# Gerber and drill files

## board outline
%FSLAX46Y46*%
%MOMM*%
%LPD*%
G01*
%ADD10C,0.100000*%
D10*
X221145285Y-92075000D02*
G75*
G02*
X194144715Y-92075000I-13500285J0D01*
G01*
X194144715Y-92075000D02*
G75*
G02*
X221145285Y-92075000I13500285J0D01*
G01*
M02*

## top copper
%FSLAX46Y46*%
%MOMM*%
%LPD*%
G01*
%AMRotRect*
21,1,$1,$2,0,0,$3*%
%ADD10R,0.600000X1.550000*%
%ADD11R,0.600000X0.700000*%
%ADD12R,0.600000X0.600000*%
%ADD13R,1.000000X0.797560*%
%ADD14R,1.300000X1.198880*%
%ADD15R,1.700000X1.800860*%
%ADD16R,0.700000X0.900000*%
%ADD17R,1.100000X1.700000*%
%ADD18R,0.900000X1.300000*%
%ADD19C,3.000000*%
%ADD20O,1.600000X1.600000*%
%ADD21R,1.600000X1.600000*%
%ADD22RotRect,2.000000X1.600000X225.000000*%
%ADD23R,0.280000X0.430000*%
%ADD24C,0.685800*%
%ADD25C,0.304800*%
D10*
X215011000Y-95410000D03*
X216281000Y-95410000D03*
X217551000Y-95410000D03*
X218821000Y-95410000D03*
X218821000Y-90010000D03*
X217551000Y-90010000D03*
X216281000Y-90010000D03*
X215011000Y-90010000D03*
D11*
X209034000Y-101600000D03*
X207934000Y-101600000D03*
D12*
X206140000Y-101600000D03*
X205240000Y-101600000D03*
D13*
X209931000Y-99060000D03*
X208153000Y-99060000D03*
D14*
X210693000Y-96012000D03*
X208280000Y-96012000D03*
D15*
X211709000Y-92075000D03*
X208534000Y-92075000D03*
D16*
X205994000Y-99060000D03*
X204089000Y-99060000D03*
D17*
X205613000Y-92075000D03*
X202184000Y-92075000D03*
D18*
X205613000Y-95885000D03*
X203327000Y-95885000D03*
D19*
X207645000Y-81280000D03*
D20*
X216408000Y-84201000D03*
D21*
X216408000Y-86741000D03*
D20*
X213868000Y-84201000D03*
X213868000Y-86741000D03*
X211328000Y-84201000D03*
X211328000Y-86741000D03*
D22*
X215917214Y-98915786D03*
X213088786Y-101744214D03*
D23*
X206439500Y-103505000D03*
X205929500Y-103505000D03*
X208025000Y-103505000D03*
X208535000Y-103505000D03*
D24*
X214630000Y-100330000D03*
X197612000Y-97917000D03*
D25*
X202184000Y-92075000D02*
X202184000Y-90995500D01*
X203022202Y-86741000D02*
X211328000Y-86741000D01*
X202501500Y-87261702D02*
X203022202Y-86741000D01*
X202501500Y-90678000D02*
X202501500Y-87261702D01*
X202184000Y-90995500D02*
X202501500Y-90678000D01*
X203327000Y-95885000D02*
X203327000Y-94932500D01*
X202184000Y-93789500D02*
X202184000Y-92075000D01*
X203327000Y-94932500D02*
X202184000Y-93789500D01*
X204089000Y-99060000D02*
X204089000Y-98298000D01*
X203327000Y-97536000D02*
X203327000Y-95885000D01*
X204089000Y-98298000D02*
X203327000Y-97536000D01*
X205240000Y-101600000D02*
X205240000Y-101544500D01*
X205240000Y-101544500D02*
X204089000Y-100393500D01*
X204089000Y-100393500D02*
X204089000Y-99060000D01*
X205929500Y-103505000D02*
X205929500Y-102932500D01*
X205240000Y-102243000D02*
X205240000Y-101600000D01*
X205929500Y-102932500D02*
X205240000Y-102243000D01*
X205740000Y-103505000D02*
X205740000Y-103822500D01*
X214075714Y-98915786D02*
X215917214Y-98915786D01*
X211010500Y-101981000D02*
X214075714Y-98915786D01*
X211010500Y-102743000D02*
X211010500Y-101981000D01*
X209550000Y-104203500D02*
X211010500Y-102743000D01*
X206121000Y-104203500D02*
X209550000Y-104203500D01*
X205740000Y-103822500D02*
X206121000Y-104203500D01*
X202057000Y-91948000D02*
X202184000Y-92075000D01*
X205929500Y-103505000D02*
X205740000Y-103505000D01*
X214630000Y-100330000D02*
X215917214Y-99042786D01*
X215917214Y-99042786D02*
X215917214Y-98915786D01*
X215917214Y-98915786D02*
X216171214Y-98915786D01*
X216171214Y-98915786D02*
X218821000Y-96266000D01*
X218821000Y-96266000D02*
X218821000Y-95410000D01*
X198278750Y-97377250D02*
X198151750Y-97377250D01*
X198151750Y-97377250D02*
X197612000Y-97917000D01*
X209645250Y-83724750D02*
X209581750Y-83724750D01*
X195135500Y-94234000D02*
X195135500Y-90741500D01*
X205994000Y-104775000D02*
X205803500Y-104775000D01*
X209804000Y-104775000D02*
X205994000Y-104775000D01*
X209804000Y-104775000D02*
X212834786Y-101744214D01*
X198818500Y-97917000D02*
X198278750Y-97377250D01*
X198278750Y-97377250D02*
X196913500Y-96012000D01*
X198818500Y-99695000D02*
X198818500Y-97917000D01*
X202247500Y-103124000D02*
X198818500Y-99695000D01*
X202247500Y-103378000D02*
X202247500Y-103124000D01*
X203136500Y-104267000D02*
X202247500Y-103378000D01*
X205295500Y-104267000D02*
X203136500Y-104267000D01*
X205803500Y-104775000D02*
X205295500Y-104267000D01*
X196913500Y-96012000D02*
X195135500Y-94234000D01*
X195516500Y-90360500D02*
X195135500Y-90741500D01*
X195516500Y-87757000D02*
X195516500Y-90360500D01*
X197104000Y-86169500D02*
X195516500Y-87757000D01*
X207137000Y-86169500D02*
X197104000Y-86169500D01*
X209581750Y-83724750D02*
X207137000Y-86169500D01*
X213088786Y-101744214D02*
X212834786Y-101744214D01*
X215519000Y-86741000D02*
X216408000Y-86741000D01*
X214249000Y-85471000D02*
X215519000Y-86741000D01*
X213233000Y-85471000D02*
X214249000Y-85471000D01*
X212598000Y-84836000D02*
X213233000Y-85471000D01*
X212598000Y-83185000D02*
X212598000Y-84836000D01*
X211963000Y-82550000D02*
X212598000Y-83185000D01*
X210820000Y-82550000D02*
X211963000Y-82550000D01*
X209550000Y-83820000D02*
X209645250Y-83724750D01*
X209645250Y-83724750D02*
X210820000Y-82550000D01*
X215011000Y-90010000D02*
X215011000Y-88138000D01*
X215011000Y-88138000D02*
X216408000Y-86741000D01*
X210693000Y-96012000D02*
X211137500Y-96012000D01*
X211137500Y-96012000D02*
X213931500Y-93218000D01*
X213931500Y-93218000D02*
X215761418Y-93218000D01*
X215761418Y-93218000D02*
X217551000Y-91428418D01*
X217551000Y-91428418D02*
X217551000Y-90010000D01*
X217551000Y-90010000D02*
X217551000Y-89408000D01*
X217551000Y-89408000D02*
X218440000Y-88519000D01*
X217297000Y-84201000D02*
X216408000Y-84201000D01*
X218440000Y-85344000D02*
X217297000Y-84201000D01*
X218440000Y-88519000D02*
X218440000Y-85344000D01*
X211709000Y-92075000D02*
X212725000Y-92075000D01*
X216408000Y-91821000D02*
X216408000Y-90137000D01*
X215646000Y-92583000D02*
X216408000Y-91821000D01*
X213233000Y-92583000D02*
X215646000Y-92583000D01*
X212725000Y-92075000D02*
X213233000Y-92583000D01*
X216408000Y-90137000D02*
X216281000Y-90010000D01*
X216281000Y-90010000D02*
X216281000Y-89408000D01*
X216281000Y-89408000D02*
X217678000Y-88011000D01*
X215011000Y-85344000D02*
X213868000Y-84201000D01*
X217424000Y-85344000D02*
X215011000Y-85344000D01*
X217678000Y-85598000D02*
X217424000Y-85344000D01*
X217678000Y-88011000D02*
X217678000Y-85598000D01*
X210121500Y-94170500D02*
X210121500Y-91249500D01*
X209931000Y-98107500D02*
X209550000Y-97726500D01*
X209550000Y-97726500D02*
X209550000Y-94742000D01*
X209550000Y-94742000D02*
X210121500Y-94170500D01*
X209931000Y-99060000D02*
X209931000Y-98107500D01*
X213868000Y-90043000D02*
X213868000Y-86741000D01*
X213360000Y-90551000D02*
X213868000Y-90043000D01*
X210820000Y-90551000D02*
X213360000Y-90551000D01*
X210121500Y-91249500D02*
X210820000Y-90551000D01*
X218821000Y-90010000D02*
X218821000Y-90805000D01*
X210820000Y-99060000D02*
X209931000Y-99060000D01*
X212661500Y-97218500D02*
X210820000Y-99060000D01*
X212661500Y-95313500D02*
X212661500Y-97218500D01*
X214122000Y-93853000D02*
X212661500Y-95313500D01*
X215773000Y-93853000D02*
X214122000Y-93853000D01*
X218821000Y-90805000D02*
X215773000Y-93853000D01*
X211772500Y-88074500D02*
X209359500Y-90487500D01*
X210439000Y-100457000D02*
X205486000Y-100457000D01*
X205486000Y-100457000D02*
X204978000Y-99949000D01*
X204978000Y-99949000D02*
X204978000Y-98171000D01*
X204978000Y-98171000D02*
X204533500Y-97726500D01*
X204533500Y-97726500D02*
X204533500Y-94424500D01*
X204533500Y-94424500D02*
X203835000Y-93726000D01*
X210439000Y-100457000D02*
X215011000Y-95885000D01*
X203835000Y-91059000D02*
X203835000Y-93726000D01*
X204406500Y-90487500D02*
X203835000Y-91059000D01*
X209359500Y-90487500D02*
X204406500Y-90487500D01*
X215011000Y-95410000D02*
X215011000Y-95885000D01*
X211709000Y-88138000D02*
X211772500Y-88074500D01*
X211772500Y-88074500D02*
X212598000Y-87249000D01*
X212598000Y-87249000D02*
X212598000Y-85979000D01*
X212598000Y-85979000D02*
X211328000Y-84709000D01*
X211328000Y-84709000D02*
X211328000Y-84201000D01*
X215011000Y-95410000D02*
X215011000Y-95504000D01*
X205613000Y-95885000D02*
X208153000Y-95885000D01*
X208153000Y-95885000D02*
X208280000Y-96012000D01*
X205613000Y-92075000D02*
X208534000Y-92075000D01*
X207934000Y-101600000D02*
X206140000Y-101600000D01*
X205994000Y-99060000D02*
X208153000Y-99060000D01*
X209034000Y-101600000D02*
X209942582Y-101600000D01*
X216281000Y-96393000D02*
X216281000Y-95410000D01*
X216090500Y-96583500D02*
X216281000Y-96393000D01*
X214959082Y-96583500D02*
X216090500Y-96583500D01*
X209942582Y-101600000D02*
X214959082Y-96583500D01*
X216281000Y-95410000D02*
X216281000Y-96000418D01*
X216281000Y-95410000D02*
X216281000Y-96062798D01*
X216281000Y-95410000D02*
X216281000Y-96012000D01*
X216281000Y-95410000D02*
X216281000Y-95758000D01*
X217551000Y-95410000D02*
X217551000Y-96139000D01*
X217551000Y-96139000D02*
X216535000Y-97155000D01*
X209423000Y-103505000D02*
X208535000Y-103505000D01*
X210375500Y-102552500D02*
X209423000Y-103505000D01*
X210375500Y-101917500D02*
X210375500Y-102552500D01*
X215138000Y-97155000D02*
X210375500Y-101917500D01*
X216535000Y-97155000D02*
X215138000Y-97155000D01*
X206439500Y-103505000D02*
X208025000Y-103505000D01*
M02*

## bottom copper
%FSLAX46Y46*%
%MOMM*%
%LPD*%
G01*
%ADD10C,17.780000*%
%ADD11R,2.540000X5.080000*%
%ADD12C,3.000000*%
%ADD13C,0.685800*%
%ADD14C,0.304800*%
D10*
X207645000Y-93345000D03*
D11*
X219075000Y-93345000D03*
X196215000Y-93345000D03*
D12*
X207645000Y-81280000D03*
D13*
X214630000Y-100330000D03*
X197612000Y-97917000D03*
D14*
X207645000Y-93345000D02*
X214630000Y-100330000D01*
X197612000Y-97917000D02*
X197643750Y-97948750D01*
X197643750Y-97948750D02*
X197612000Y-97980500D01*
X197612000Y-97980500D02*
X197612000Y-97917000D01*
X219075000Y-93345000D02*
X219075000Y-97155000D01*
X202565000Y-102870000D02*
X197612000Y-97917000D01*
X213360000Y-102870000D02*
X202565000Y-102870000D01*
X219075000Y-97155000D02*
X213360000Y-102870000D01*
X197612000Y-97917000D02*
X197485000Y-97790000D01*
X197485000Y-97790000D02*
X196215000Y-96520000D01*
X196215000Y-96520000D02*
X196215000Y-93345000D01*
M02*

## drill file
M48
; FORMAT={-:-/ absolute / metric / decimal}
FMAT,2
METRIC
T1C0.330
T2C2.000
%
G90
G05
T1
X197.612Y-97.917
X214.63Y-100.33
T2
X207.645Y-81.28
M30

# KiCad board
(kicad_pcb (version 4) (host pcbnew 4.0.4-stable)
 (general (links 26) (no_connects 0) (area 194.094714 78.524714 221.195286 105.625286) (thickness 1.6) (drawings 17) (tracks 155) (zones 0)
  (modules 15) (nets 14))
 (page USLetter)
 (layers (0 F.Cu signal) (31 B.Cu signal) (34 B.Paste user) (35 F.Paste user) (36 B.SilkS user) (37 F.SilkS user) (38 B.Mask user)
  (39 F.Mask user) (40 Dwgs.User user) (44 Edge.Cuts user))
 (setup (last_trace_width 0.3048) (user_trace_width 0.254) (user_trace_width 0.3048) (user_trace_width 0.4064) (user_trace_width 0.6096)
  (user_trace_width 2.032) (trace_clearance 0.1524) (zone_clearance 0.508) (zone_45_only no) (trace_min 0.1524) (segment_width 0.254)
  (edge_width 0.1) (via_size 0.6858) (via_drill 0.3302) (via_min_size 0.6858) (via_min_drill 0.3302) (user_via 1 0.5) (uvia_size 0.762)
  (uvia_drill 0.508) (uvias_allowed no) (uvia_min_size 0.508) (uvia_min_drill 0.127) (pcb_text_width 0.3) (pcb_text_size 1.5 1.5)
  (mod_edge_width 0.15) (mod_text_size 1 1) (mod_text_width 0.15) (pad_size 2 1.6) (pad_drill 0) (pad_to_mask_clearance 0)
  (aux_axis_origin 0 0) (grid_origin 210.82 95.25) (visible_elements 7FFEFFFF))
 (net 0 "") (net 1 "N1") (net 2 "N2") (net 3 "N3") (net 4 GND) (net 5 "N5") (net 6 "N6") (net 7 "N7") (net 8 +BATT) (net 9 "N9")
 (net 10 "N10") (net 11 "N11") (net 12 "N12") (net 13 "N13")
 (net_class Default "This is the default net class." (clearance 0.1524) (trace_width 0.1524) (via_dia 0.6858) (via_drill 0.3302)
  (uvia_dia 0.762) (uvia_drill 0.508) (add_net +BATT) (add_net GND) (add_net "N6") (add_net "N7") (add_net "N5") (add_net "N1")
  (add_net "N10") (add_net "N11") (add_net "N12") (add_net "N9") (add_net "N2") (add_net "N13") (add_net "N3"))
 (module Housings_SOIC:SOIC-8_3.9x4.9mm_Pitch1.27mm (layer F.Cu) (at 216.916 92.71 90)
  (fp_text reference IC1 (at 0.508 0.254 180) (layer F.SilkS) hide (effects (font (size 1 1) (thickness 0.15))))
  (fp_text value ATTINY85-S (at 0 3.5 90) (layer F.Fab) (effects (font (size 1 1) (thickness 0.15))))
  (pad 1 smd rect (at -2.7 -1.905 90) (size 1.55 0.6) (layers F.Cu F.Paste F.Mask) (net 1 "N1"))
  (pad 2 smd rect (at -2.7 -0.635 90) (size 1.55 0.6) (layers F.Cu F.Paste F.Mask) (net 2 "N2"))
  (pad 3 smd rect (at -2.7 0.635 90) (size 1.55 0.6) (layers F.Cu F.Paste F.Mask) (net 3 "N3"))
  (pad 4 smd rect (at -2.7 1.905 90) (size 1.55 0.6) (layers F.Cu F.Paste F.Mask) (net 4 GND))
  (pad 5 smd rect (at 2.7 1.905 90) (size 1.55 0.6) (layers F.Cu F.Paste F.Mask) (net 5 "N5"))
  (pad 6 smd rect (at 2.7 0.635 90) (size 1.55 0.6) (layers F.Cu F.Paste F.Mask) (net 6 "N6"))
  (pad 7 smd rect (at 2.7 -0.635 90) (size 1.55 0.6) (layers F.Cu F.Paste F.Mask) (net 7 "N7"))
  (pad 8 smd rect (at 2.7 -1.905 90) (size 1.55 0.6) (layers F.Cu F.Paste F.Mask) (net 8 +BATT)))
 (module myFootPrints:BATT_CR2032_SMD (layer B.Cu) (at 207.645 93.345 180)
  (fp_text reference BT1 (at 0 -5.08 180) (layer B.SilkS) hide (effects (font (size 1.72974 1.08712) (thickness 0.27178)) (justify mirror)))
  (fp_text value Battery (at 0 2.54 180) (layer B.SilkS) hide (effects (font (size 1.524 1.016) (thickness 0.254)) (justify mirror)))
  (pad 2 smd circle (at 0 0 180) (size 17.78 17.78) (layers B.Cu B.Paste B.Mask) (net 4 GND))
  (pad 1 smd rect (at -11.43 0 180) (size 2.54 5.08) (layers B.Cu B.Paste B.Mask) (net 8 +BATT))
  (pad 1 smd rect (at 11.43 0 180) (size 2.54 5.08) (layers B.Cu B.Paste B.Mask) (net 8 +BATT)))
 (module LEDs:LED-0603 (layer F.Cu) (at 208.534 101.6)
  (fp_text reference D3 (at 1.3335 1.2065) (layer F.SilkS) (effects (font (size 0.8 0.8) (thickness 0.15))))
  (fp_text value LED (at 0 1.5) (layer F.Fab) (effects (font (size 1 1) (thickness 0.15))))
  (pad 2 smd rect (at 0.5 0 180) (size 0.6 0.7) (layers F.Cu F.Paste F.Mask) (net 2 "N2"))
  (pad 1 smd rect (at -0.6 0 180) (size 0.6 0.7) (layers F.Cu F.Paste F.Mask) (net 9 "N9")))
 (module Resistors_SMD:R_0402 (layer F.Cu) (at 205.74 101.6 180)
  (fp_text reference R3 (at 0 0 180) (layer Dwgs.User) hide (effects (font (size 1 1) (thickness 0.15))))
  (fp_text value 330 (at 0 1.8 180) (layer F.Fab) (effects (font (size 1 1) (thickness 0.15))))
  (pad 1 smd rect (at -0.4 0 180) (size 0.6 0.6) (layers F.Cu F.Paste F.Mask) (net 9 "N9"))
  (pad 2 smd rect (at 0.5 0 180) (size 0.6 0.6) (layers F.Cu F.Paste F.Mask) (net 4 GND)))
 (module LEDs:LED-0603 (layer F.Cu) (at 209.042 99.06)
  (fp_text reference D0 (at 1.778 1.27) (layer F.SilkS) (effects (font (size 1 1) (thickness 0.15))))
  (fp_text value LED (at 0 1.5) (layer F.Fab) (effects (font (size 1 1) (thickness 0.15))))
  (pad 2 smd rect (at 0.889 0 180) (size 1 0.79756) (layers F.Cu F.Paste F.Mask) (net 5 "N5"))
  (pad 1 smd rect (at -0.889 0 180) (size 1 0.79756) (layers F.Cu F.Paste F.Mask) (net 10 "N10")))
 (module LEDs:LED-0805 (layer F.Cu) (at 209.55 96.012)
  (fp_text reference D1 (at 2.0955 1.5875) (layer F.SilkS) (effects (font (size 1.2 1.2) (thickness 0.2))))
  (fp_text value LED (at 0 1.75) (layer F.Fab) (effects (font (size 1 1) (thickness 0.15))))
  (pad 2 smd rect (at 1.143 0 180) (size 1.3 1.19888) (layers F.Cu F.Paste F.Mask) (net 6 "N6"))
  (pad 1 smd rect (at -1.27 0 180) (size 1.3 1.19888) (layers F.Cu F.Paste F.Mask) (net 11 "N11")))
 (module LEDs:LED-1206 (layer F.Cu) (at 210.185 92.075)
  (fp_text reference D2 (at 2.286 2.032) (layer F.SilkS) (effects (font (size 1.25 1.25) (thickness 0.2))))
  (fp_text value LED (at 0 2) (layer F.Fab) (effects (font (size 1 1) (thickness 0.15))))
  (pad 2 smd rect (at 1.524 0 180) (size 1.7 1.80086) (layers F.Cu F.Paste F.Mask) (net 7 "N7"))
  (pad 1 smd rect (at -1.651 0 180) (size 1.7 1.80086) (layers F.Cu F.Paste F.Mask) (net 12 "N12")))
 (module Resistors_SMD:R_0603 (layer F.Cu) (at 205.105 99.06 180)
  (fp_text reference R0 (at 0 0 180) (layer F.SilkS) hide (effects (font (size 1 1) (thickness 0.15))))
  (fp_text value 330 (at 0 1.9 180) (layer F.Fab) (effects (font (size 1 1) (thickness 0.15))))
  (pad 1 smd rect (at -0.889 0 180) (size 0.7 0.9) (layers F.Cu F.Paste F.Mask) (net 10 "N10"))
  (pad 2 smd rect (at 1.016 0 180) (size 0.7 0.9) (layers F.Cu F.Paste F.Mask) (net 4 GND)))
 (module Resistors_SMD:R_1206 (layer F.Cu) (at 203.835 92.075 180)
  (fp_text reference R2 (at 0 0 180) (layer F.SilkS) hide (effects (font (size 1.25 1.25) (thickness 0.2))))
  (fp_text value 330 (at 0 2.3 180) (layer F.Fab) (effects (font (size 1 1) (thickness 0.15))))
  (pad 1 smd rect (at -1.778 0 180) (size 1.1 1.7) (layers F.Cu F.Paste F.Mask) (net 12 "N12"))
  (pad 2 smd rect (at 1.651 0 180) (size 1.1 1.7) (layers F.Cu F.Paste F.Mask) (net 4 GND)))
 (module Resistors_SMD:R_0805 (layer F.Cu) (at 204.47 95.885 180)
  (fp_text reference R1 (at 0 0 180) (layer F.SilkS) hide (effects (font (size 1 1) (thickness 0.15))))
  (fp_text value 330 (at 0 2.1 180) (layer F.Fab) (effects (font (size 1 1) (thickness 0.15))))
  (pad 1 smd rect (at -1.143 0 180) (size 0.9 1.3) (layers F.Cu F.Paste F.Mask) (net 11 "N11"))
  (pad 2 smd rect (at 1.143 0 180) (size 0.9 1.3) (layers F.Cu F.Paste F.Mask) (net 4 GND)))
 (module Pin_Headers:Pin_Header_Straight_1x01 (layer F.Cu) (at 207.645 81.28)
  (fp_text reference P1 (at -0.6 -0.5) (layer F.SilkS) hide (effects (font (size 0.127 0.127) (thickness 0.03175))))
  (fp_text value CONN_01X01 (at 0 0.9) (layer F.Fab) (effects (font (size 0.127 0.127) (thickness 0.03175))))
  (pad "" thru_hole circle (at 0 0) (size 3 3) (drill 2) (layers *.Cu *.Mask)))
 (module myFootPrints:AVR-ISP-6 (layer F.Cu) (at 216.408 84.201 270)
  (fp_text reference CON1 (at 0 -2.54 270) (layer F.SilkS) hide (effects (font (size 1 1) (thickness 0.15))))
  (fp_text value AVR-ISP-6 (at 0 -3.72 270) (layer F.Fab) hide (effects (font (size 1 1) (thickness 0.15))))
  (pad 1 smd oval (at 0 0 270) (size 1.6 1.6) (layers F.Cu F.Paste F.Mask) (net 6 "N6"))
  (pad 2 smd rect (at 2.54 0 270) (size 1.6 1.6) (layers F.Cu F.Paste F.Mask) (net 8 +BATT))
  (pad 3 smd oval (at 0 2.54 270) (size 1.6 1.6) (layers F.Cu F.Paste F.Mask) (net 7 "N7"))
  (pad 4 smd oval (at 2.54 2.54 270) (size 1.6 1.6) (layers F.Cu F.Paste F.Mask) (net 5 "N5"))
  (pad 5 smd oval (at 0 5.08 270) (size 1.6 1.6) (layers F.Cu F.Paste F.Mask) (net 1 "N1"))
  (pad 6 smd oval (at 2.54 5.08 270) (size 1.6 1.6) (layers F.Cu F.Paste F.Mask) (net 4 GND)))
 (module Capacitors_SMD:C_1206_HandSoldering (layer F.Cu) (at 214.503 100.33 225)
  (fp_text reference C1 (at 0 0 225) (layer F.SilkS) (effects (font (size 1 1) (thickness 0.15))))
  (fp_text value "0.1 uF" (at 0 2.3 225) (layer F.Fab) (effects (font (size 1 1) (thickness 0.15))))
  (pad 1 smd rect (at -2 0 225) (size 2 1.6) (layers F.Cu F.Paste F.Mask) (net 4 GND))
  (pad 2 smd rect (at 2 0 225) (size 2 1.6) (layers F.Cu F.Paste F.Mask) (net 8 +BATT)))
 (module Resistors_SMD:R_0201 (layer F.Cu) (at 206.1845 103.505 180)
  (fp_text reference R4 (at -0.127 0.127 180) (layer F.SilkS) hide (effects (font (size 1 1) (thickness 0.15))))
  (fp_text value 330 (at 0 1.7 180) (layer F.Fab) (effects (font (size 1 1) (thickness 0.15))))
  (pad 1 smd rect (at -0.255 0 180) (size 0.28 0.43) (layers F.Cu F.Paste F.Mask) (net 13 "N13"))
  (pad 2 smd rect (at 0.255 0 180) (size 0.28 0.43) (layers F.Cu F.Paste F.Mask) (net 4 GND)))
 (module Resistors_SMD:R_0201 (layer F.Cu) (at 208.28 103.505)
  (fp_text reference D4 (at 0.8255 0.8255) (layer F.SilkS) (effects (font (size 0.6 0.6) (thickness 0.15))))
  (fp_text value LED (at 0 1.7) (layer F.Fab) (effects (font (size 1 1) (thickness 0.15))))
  (pad 1 smd rect (at -0.255 0) (size 0.28 0.43) (layers F.Cu F.Paste F.Mask) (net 13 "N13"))
  (pad 2 smd rect (at 0.255 0) (size 0.28 0.43) (layers F.Cu F.Paste F.Mask) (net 3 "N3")))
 (gr_circle (center 207.645 92.075) (end 197.485 83.185) (layer Edge.Cuts) (width 0.1))
 (segment (start 202.184 92.075) (end 202.184 90.9955) (width 0.3048) (layer F.Cu) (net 4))
 (segment (start 203.022202 86.741) (end 211.328 86.741) (width 0.3048) (layer F.Cu) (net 4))
 (segment (start 202.5015 87.261702) (end 203.022202 86.741) (width 0.3048) (layer F.Cu) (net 4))
 (segment (start 202.5015 90.678) (end 202.5015 87.261702) (width 0.3048) (layer F.Cu) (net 4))
 (segment (start 202.184 90.9955) (end 202.5015 90.678) (width 0.3048) (layer F.Cu) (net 4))
 (segment (start 203.327 95.885) (end 203.327 94.9325) (width 0.3048) (layer F.Cu) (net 4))
 (segment (start 202.184 93.7895) (end 202.184 92.075) (width 0.3048) (layer F.Cu) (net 4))
 (segment (start 203.327 94.9325) (end 202.184 93.7895) (width 0.3048) (layer F.Cu) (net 4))
 (segment (start 204.089 99.06) (end 204.089 98.298) (width 0.3048) (layer F.Cu) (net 4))
 (segment (start 203.327 97.536) (end 203.327 95.885) (width 0.3048) (layer F.Cu) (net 4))
 (segment (start 204.089 98.298) (end 203.327 97.536) (width 0.3048) (layer F.Cu) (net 4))
 (segment (start 205.24 101.6) (end 205.24 101.5445) (width 0.3048) (layer F.Cu) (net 4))
 (segment (start 205.24 101.5445) (end 204.089 100.3935) (width 0.3048) (layer F.Cu) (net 4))
 (segment (start 204.089 100.3935) (end 204.089 99.06) (width 0.3048) (layer F.Cu) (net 4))
 (segment (start 205.9295 103.505) (end 205.9295 102.9325) (width 0.3048) (layer F.Cu) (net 4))
 (segment (start 205.24 102.243) (end 205.24 101.6) (width 0.3048) (layer F.Cu) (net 4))
 (segment (start 205.9295 102.9325) (end 205.24 102.243) (width 0.3048) (layer F.Cu) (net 4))
 (segment (start 205.74 103.505) (end 205.74 103.8225) (width 0.3048) (layer F.Cu) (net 4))
 (segment (start 214.075714 98.915786) (end 215.917214 98.915786) (width 0.3048) (layer F.Cu) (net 4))
 (segment (start 211.0105 101.981) (end 214.075714 98.915786) (width 0.3048) (layer F.Cu) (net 4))
 (segment (start 211.0105 102.743) (end 211.0105 101.981) (width 0.3048) (layer F.Cu) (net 4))
 (segment (start 209.55 104.2035) (end 211.0105 102.743) (width 0.3048) (layer F.Cu) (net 4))
 (segment (start 206.121 104.2035) (end 209.55 104.2035) (width 0.3048) (layer F.Cu) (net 4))
 (segment (start 205.74 103.8225) (end 206.121 104.2035) (width 0.3048) (layer F.Cu) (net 4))
 (segment (start 202.057 91.948) (end 202.184 92.075) (width 0.3048) (layer F.Cu) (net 4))
 (segment (start 205.9295 103.505) (end 205.74 103.505) (width 0.3048) (layer F.Cu) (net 4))
 (segment (start 207.645 93.345) (end 214.63 100.33) (width 0.3048) (layer B.Cu) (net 4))
 (segment (start 214.63 100.33) (end 215.917214 99.042786) (width 0.3048) (layer F.Cu) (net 4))
 (via (at 214.63 100.33) (size 0.6858) (drill 0.3302) (layers F.Cu B.Cu) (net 4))
 (segment (start 215.917214 99.042786) (end 215.917214 98.915786) (width 0.3048) (layer F.Cu) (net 4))
 (segment (start 215.917214 98.915786) (end 216.171214 98.915786) (width 0.3048) (layer F.Cu) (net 4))
 (segment (start 216.171214 98.915786) (end 218.821 96.266) (width 0.3048) (layer F.Cu) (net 4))
 (segment (start 218.821 96.266) (end 218.821 95.41) (width 0.3048) (layer F.Cu) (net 4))
 (segment (start 198.27875 97.37725) (end 198.15175 97.37725) (width 0.3048) (layer F.Cu) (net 8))
 (via (at 197.612 97.917) (size 0.6858) (drill 0.3302) (layers F.Cu B.Cu) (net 8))
 (segment (start 198.15175 97.37725) (end 197.612 97.917) (width 0.3048) (layer F.Cu) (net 8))
 (segment (start 197.612 97.917) (end 197.64375 97.94875) (width 0.3048) (layer B.Cu) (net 8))
 (segment (start 197.64375 97.94875) (end 197.612 97.9805) (width 0.3048) (layer B.Cu) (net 8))
 (segment (start 197.612 97.9805) (end 197.612 97.917) (width 0.3048) (layer B.Cu) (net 8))
 (segment (start 209.64525 83.72475) (end 209.58175 83.72475) (width 0.3048) (layer F.Cu) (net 8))
 (segment (start 195.1355 94.234) (end 195.1355 90.7415) (width 0.3048) (layer F.Cu) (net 8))
 (segment (start 205.994 104.775) (end 205.8035 104.775) (width 0.3048) (layer F.Cu) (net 8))
 (segment (start 209.804 104.775) (end 205.994 104.775) (width 0.3048) (layer F.Cu) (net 8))
 (segment (start 209.804 104.775) (end 212.834786 101.744214) (width 0.3048) (layer F.Cu) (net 8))
 (segment (start 198.8185 97.917) (end 198.27875 97.37725) (width 0.3048) (layer F.Cu) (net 8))
 (segment (start 198.27875 97.37725) (end 196.9135 96.012) (width 0.3048) (layer F.Cu) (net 8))
 (segment (start 198.8185 99.695) (end 198.8185 97.917) (width 0.3048) (layer F.Cu) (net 8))
 (segment (start 202.2475 103.124) (end 198.8185 99.695) (width 0.3048) (layer F.Cu) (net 8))
 (segment (start 202.2475 103.378) (end 202.2475 103.124) (width 0.3048) (layer F.Cu) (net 8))
 (segment (start 203.1365 104.267) (end 202.2475 103.378) (width 0.3048) (layer F.Cu) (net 8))
 (segment (start 205.2955 104.267) (end 203.1365 104.267) (width 0.3048) (layer F.Cu) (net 8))
 (segment (start 205.8035 104.775) (end 205.2955 104.267) (width 0.3048) (layer F.Cu) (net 8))
 (segment (start 196.9135 96.012) (end 195.1355 94.234) (width 0.3048) (layer F.Cu) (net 8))
 (segment (start 195.5165 90.3605) (end 195.1355 90.7415) (width 0.3048) (layer F.Cu) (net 8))
 (segment (start 195.5165 87.757) (end 195.5165 90.3605) (width 0.3048) (layer F.Cu) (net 8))
 (segment (start 197.104 86.1695) (end 195.5165 87.757) (width 0.3048) (layer F.Cu) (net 8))
 (segment (start 207.137 86.1695) (end 197.104 86.1695) (width 0.3048) (layer F.Cu) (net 8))
 (segment (start 209.58175 83.72475) (end 207.137 86.1695) (width 0.3048) (layer F.Cu) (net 8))
 (segment (start 219.075 93.345) (end 219.075 97.155) (width 0.3048) (layer B.Cu) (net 8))
 (segment (start 202.565 102.87) (end 197.612 97.917) (width 0.3048) (layer B.Cu) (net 8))
 (segment (start 213.36 102.87) (end 202.565 102.87) (width 0.3048) (layer B.Cu) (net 8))
 (segment (start 219.075 97.155) (end 213.36 102.87) (width 0.3048) (layer B.Cu) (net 8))
 (segment (start 197.612 97.917) (end 197.485 97.79) (width 0.3048) (layer B.Cu) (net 8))
 (segment (start 197.485 97.79) (end 196.215 96.52) (width 0.3048) (layer B.Cu) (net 8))
 (segment (start 196.215 96.52) (end 196.215 93.345) (width 0.3048) (layer B.Cu) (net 8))
 (segment (start 213.088786 101.744214) (end 212.834786 101.744214) (width 0.3048) (layer F.Cu) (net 8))
 (segment (start 215.519 86.741) (end 216.408 86.741) (width 0.3048) (layer F.Cu) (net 8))
 (segment (start 214.249 85.471) (end 215.519 86.741) (width 0.3048) (layer F.Cu) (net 8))
 (segment (start 213.233 85.471) (end 214.249 85.471) (width 0.3048) (layer F.Cu) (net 8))
 (segment (start 212.598 84.836) (end 213.233 85.471) (width 0.3048) (layer F.Cu) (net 8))
 (segment (start 212.598 83.185) (end 212.598 84.836) (width 0.3048) (layer F.Cu) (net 8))
 (segment (start 211.963 82.55) (end 212.598 83.185) (width 0.3048) (layer F.Cu) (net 8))
 (segment (start 210.82 82.55) (end 211.963 82.55) (width 0.3048) (layer F.Cu) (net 8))
 (segment (start 209.55 83.82) (end 209.64525 83.72475) (width 0.3048) (layer F.Cu) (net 8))
 (segment (start 209.64525 83.72475) (end 210.82 82.55) (width 0.3048) (layer F.Cu) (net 8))
 (segment (start 215.011 90.01) (end 215.011 88.138) (width 0.3048) (layer F.Cu) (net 8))
 (segment (start 215.011 88.138) (end 216.408 86.741) (width 0.3048) (layer F.Cu) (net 8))
 (segment (start 210.693 96.012) (end 211.1375 96.012) (width 0.3048) (layer F.Cu) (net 6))
 (segment (start 211.1375 96.012) (end 213.9315 93.218) (width 0.3048) (layer F.Cu) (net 6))
 (segment (start 213.9315 93.218) (end 215.761418 93.218) (width 0.3048) (layer F.Cu) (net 6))
 (segment (start 215.761418 93.218) (end 217.551 91.428418) (width 0.3048) (layer F.Cu) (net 6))
 (segment (start 217.551 91.428418) (end 217.551 90.01) (width 0.3048) (layer F.Cu) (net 6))
 (segment (start 217.551 90.01) (end 217.551 89.408) (width 0.3048) (layer F.Cu) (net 6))
 (segment (start 217.551 89.408) (end 218.44 88.519) (width 0.3048) (layer F.Cu) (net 6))
 (segment (start 217.297 84.201) (end 216.408 84.201) (width 0.3048) (layer F.Cu) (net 6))
 (segment (start 218.44 85.344) (end 217.297 84.201) (width 0.3048) (layer F.Cu) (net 6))
 (segment (start 218.44 88.519) (end 218.44 85.344) (width 0.3048) (layer F.Cu) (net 6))
 (segment (start 211.709 92.075) (end 212.725 92.075) (width 0.3048) (layer F.Cu) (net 7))
 (segment (start 216.408 91.821) (end 216.408 90.137) (width 0.3048) (layer F.Cu) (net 7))
 (segment (start 215.646 92.583) (end 216.408 91.821) (width 0.3048) (layer F.Cu) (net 7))
 (segment (start 213.233 92.583) (end 215.646 92.583) (width 0.3048) (layer F.Cu) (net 7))
 (segment (start 212.725 92.075) (end 213.233 92.583) (width 0.3048) (layer F.Cu) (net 7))
 (segment (start 216.408 90.137) (end 216.281 90.01) (width 0.3048) (layer F.Cu) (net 7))
 (segment (start 216.281 90.01) (end 216.281 89.408) (width 0.3048) (layer F.Cu) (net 7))
 (segment (start 216.281 89.408) (end 217.678 88.011) (width 0.3048) (layer F.Cu) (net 7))
 (segment (start 215.011 85.344) (end 213.868 84.201) (width 0.3048) (layer F.Cu) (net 7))
 (segment (start 217.424 85.344) (end 215.011 85.344) (width 0.3048) (layer F.Cu) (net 7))
 (segment (start 217.678 85.598) (end 217.424 85.344) (width 0.3048) (layer F.Cu) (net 7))
 (segment (start 217.678 88.011) (end 217.678 85.598) (width 0.3048) (layer F.Cu) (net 7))
 (segment (start 210.1215 94.1705) (end 210.1215 91.2495) (width 0.3048) (layer F.Cu) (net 5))
 (segment (start 209.931 98.1075) (end 209.55 97.7265) (width 0.3048) (layer F.Cu) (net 5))
 (segment (start 209.55 97.7265) (end 209.55 94.742) (width 0.3048) (layer F.Cu) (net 5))
 (segment (start 209.55 94.742) (end 210.1215 94.1705) (width 0.3048) (layer F.Cu) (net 5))
 (segment (start 209.931 99.06) (end 209.931 98.1075) (width 0.3048) (layer F.Cu) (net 5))
 (segment (start 213.868 90.043) (end 213.868 86.741) (width 0.3048) (layer F.Cu) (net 5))
 (segment (start 213.36 90.551) (end 213.868 90.043) (width 0.3048) (layer F.Cu) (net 5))
 (segment (start 210.82 90.551) (end 213.36 90.551) (width 0.3048) (layer F.Cu) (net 5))
 (segment (start 210.1215 91.2495) (end 210.82 90.551) (width 0.3048) (layer F.Cu) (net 5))
 (segment (start 218.821 90.01) (end 218.821 90.805) (width 0.3048) (layer F.Cu) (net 5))
 (segment (start 210.82 99.06) (end 209.931 99.06) (width 0.3048) (layer F.Cu) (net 5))
 (segment (start 212.6615 97.2185) (end 210.82 99.06) (width 0.3048) (layer F.Cu) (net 5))
 (segment (start 212.6615 95.3135) (end 212.6615 97.2185) (width 0.3048) (layer F.Cu) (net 5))
 (segment (start 214.122 93.853) (end 212.6615 95.3135) (width 0.3048) (layer F.Cu) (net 5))
 (segment (start 215.773 93.853) (end 214.122 93.853) (width 0.3048) (layer F.Cu) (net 5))
 (segment (start 218.821 90.805) (end 215.773 93.853) (width 0.3048) (layer F.Cu) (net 5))
 (segment (start 211.7725 88.0745) (end 209.3595 90.4875) (width 0.3048) (layer F.Cu) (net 1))
 (segment (start 210.439 100.457) (end 205.486 100.457) (width 0.3048) (layer F.Cu) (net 1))
 (segment (start 205.486 100.457) (end 204.978 99.949) (width 0.3048) (layer F.Cu) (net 1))
 (segment (start 204.978 99.949) (end 204.978 98.171) (width 0.3048) (layer F.Cu) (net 1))
 (segment (start 204.978 98.171) (end 204.5335 97.7265) (width 0.3048) (layer F.Cu) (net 1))
 (segment (start 204.5335 97.7265) (end 204.5335 94.4245) (width 0.3048) (layer F.Cu) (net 1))
 (segment (start 204.5335 94.4245) (end 203.835 93.726) (width 0.3048) (layer F.Cu) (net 1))
 (segment (start 210.439 100.457) (end 215.011 95.885) (width 0.3048) (layer F.Cu) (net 1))
 (segment (start 203.835 91.059) (end 203.835 93.726) (width 0.3048) (layer F.Cu) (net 1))
 (segment (start 204.4065 90.4875) (end 203.835 91.059) (width 0.3048) (layer F.Cu) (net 1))
 (segment (start 209.3595 90.4875) (end 204.4065 90.4875) (width 0.3048) (layer F.Cu) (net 1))
 (segment (start 215.011 95.41) (end 215.011 95.885) (width 0.3048) (layer F.Cu) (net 1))
 (segment (start 211.709 88.138) (end 211.7725 88.0745) (width 0.3048) (layer F.Cu) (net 1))
 (segment (start 211.7725 88.0745) (end 212.598 87.249) (width 0.3048) (layer F.Cu) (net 1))
 (segment (start 212.598 87.249) (end 212.598 85.979) (width 0.3048) (layer F.Cu) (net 1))
 (segment (start 212.598 85.979) (end 211.328 84.709) (width 0.3048) (layer F.Cu) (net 1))
 (segment (start 211.328 84.709) (end 211.328 84.201) (width 0.3048) (layer F.Cu) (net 1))
 (segment (start 215.011 95.41) (end 215.011 95.504) (width 0.3048) (layer F.Cu) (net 1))
 (segment (start 205.613 95.885) (end 208.153 95.885) (width 0.3048) (layer F.Cu) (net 11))
 (segment (start 208.153 95.885) (end 208.28 96.012) (width 0.3048) (layer F.Cu) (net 11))
 (segment (start 205.613 92.075) (end 208.534 92.075) (width 0.3048) (layer F.Cu) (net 12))
 (segment (start 207.934 101.6) (end 206.14 101.6) (width 0.3048) (layer F.Cu) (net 9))
 (segment (start 205.994 99.06) (end 208.153 99.06) (width 0.3048) (layer F.Cu) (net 10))
 (segment (start 209.034 101.6) (end 209.942582 101.6) (width 0.3048) (layer F.Cu) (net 2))
 (segment (start 216.281 96.393) (end 216.281 95.41) (width 0.3048) (layer F.Cu) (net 2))
 (segment (start 216.0905 96.5835) (end 216.281 96.393) (width 0.3048) (layer F.Cu) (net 2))
 (segment (start 214.959082 96.5835) (end 216.0905 96.5835) (width 0.3048) (layer F.Cu) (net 2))
 (segment (start 209.942582 101.6) (end 214.959082 96.5835) (width 0.3048) (layer F.Cu) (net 2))
 (segment (start 216.281 95.41) (end 216.281 96.000418) (width 0.3048) (layer F.Cu) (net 2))
 (segment (start 216.281 95.41) (end 216.281 96.062798) (width 0.3048) (layer F.Cu) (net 2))
 (segment (start 216.281 95.41) (end 216.281 96.012) (width 0.3048) (layer F.Cu) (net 2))
 (segment (start 216.281 95.41) (end 216.281 95.758) (width 0.3048) (layer F.Cu) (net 2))
 (segment (start 217.551 95.41) (end 217.551 96.139) (width 0.3048) (layer F.Cu) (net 3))
 (segment (start 217.551 96.139) (end 216.535 97.155) (width 0.3048) (layer F.Cu) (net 3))
 (segment (start 209.423 103.505) (end 208.535 103.505) (width 0.3048) (layer F.Cu) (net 3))
 (segment (start 210.3755 102.5525) (end 209.423 103.505) (width 0.3048) (layer F.Cu) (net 3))
 (segment (start 210.3755 101.9175) (end 210.3755 102.5525) (width 0.3048) (layer F.Cu) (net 3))
 (segment (start 215.138 97.155) (end 210.3755 101.9175) (width 0.3048) (layer F.Cu) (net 3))
 (segment (start 216.535 97.155) (end 215.138 97.155) (width 0.3048) (layer F.Cu) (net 3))
 (segment (start 206.4395 103.505) (end 208.025 103.505) (width 0.3048) (layer F.Cu) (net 13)))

